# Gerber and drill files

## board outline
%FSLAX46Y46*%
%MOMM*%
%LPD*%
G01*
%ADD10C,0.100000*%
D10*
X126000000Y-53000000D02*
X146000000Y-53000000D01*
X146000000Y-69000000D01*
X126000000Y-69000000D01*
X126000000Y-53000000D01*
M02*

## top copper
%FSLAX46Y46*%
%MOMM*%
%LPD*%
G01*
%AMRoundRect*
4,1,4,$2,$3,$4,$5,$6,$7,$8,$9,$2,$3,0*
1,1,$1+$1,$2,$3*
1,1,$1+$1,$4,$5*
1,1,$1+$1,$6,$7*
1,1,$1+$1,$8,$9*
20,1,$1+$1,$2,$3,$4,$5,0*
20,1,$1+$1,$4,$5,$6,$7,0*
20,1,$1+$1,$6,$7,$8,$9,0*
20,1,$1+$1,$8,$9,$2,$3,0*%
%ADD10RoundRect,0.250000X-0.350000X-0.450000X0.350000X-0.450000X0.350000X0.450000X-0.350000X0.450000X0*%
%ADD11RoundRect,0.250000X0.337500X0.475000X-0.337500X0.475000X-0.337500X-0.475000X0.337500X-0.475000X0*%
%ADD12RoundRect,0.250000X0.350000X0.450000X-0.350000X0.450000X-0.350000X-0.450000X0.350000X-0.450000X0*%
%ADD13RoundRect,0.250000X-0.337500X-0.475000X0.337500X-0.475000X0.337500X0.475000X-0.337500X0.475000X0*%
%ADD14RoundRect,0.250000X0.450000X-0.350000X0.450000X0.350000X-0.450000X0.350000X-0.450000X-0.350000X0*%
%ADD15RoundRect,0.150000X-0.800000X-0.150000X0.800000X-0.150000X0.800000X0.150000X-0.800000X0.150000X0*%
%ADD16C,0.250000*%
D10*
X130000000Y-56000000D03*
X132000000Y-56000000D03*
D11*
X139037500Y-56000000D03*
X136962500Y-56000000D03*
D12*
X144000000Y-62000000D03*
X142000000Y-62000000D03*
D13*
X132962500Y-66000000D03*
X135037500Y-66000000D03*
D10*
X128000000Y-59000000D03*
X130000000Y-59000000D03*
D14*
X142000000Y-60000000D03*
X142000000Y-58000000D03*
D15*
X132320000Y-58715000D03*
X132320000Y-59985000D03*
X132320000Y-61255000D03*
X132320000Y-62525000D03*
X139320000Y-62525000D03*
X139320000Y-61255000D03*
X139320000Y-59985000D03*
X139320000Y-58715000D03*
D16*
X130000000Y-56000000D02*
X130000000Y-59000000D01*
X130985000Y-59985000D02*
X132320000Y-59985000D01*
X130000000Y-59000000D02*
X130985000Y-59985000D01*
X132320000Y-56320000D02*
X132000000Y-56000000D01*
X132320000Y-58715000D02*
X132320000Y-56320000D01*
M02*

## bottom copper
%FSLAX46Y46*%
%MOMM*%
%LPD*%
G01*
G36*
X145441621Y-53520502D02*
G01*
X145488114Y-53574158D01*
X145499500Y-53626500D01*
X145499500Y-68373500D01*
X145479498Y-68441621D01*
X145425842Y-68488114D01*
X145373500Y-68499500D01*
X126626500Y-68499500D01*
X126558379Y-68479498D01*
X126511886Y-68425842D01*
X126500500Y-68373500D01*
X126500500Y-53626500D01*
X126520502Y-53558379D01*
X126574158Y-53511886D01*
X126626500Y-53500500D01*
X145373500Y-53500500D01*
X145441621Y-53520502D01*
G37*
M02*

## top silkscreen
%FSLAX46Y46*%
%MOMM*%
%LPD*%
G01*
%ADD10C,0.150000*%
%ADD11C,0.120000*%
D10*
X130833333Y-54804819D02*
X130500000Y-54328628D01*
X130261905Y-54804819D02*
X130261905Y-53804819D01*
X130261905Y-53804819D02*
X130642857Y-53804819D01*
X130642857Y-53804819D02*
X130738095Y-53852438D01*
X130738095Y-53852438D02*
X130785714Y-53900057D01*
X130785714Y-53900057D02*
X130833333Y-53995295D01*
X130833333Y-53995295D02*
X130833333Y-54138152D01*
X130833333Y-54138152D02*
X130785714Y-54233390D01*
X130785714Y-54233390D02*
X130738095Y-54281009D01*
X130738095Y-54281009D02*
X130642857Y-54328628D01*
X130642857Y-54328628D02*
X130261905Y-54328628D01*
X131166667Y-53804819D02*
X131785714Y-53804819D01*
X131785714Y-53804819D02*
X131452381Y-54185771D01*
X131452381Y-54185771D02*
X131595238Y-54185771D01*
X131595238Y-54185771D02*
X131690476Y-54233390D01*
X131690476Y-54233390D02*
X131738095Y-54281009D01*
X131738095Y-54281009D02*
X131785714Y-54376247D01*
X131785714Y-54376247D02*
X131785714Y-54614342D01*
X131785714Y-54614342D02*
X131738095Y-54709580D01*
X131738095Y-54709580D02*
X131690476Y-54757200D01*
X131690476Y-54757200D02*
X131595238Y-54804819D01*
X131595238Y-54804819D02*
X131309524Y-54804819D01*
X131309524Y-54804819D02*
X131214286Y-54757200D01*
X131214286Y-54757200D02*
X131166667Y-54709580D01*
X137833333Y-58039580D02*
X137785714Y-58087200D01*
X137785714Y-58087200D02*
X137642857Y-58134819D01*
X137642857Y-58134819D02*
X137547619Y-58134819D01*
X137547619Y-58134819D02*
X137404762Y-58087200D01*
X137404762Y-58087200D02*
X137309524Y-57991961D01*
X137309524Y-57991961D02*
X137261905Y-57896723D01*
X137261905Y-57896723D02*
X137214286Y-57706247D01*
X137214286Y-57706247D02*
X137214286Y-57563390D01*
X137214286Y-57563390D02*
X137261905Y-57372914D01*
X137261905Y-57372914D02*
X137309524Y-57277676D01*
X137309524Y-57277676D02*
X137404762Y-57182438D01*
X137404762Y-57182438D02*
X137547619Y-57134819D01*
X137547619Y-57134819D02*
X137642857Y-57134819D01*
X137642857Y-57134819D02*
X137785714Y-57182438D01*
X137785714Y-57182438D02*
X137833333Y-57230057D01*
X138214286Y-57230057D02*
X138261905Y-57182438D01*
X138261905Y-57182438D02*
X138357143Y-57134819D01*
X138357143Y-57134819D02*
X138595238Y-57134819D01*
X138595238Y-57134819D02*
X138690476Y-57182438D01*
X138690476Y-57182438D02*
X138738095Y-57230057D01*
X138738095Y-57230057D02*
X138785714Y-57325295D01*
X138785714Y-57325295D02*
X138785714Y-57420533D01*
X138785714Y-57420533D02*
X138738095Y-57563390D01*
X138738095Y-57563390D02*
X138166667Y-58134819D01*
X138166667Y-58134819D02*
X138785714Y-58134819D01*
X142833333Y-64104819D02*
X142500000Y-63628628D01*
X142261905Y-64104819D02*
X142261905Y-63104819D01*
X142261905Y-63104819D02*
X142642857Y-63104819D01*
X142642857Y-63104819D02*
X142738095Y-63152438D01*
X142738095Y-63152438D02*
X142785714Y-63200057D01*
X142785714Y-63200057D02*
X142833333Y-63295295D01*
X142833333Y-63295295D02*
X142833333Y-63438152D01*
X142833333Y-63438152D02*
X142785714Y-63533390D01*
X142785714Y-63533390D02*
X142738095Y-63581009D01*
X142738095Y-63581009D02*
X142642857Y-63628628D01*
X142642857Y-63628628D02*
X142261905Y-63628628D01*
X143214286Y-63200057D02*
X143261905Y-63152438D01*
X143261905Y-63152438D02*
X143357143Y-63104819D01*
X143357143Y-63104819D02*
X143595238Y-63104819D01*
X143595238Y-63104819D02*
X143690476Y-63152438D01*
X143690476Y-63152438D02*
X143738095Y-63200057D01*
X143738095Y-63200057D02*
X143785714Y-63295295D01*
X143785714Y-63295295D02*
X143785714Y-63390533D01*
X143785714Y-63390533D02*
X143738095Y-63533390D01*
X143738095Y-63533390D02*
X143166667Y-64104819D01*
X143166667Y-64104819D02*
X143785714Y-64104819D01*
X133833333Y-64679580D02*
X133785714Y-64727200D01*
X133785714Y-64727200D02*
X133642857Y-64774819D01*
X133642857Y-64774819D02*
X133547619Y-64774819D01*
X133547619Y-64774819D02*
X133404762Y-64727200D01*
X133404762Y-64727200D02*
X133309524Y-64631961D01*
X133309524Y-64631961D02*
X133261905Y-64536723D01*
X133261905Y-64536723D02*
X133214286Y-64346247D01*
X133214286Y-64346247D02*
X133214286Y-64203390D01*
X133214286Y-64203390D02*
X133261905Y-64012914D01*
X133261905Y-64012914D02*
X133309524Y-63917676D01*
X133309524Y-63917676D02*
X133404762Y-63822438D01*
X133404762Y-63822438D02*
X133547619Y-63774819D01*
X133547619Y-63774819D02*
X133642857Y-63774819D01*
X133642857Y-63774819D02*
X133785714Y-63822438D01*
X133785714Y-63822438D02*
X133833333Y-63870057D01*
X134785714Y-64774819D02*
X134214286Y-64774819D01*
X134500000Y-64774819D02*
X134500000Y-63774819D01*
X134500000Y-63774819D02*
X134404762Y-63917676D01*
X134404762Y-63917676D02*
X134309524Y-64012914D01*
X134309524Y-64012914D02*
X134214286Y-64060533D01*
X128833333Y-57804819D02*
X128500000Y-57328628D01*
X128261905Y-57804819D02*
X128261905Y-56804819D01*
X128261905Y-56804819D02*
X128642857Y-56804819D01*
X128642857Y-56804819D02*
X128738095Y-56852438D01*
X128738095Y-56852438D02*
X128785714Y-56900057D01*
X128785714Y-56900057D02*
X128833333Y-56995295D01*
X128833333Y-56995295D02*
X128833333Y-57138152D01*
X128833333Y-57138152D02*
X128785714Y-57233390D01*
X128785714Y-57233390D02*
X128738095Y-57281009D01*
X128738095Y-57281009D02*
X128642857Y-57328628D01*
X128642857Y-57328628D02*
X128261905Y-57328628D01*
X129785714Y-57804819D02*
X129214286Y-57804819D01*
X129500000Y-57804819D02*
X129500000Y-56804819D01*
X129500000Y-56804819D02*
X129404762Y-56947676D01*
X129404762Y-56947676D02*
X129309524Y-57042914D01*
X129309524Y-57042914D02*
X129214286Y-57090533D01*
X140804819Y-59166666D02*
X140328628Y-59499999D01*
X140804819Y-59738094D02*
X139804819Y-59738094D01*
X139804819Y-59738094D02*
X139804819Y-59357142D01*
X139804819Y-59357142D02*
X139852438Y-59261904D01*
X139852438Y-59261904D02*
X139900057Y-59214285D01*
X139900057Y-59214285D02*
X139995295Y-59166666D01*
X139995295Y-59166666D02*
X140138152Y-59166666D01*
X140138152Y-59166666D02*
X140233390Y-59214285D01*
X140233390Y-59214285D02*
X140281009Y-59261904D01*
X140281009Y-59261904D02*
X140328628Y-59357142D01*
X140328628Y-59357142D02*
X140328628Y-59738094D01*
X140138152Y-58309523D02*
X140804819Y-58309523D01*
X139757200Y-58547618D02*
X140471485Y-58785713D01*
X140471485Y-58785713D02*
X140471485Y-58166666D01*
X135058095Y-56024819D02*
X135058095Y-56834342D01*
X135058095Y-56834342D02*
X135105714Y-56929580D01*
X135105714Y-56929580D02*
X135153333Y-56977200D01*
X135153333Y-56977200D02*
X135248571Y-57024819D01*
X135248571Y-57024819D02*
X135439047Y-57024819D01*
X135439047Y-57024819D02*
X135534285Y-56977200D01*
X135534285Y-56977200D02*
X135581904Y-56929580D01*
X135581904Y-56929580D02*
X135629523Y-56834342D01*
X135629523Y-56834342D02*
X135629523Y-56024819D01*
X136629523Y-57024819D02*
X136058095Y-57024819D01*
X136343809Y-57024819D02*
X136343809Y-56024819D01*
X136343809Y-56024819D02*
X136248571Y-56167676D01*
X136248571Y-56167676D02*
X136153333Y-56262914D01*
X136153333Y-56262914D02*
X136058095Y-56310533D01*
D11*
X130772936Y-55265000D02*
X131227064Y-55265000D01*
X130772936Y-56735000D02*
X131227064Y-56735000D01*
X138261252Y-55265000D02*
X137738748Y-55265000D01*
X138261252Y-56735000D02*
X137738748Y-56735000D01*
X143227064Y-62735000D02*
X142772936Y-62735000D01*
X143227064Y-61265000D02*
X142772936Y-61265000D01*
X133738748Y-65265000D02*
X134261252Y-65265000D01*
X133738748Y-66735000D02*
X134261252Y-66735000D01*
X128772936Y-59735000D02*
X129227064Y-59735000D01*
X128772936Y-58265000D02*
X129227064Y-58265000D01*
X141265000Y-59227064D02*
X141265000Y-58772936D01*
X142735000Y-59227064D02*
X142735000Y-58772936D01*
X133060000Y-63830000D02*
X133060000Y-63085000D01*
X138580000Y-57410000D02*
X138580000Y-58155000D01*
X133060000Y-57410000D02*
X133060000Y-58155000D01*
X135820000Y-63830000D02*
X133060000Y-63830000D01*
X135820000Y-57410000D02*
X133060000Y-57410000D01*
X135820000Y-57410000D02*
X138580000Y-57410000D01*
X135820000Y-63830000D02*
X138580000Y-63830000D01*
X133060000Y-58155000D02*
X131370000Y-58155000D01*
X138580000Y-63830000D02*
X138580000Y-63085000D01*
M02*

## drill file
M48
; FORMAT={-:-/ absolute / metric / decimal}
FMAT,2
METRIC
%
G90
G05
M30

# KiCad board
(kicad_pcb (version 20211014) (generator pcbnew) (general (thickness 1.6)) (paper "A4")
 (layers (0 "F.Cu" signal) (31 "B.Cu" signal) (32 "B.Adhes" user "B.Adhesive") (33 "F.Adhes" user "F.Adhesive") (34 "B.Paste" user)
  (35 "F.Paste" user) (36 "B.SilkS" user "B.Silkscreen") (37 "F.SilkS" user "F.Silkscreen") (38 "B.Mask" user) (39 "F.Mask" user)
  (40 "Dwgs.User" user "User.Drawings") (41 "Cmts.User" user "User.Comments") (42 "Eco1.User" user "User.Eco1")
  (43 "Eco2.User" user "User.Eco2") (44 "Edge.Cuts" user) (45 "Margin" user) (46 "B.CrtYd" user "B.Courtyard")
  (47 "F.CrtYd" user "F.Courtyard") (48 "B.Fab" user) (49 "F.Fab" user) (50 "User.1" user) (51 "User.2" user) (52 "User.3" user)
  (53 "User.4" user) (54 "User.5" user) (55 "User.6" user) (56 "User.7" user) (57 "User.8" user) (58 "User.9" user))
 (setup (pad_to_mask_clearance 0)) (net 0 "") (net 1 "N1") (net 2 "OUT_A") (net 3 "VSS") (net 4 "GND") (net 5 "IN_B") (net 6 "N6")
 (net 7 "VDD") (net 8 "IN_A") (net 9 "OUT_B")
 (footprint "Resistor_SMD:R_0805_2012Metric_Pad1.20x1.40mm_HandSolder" (layer "F.Cu") (at 131 56)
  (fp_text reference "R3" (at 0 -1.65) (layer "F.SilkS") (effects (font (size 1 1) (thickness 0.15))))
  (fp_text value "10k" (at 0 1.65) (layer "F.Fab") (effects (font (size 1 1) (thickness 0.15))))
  (fp_line (start -0.227064 -0.735) (end 0.227064 -0.735) (layer "F.SilkS") (width 0.12))
  (fp_line (start -0.227064 0.735) (end 0.227064 0.735) (layer "F.SilkS") (width 0.12))
  (pad "1" smd roundrect (at -1 0) (size 1.2 1.4) (layers "F.Cu" "F.Paste" "F.Mask") (roundrect_rratio 0.208333) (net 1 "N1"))
  (pad "2" smd roundrect (at 1 0) (size 1.2 1.4) (layers "F.Cu" "F.Paste" "F.Mask") (roundrect_rratio 0.208333) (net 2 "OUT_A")))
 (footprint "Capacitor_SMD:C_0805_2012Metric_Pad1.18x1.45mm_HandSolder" (layer "F.Cu") (at 138 56 180)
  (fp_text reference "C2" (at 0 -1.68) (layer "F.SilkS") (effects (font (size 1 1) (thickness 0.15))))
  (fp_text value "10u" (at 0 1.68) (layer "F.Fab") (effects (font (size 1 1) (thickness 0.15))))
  (fp_line (start -0.261252 0.735) (end 0.261252 0.735) (layer "F.SilkS") (width 0.12))
  (fp_line (start -0.261252 -0.735) (end 0.261252 -0.735) (layer "F.SilkS") (width 0.12))
  (pad "1" smd roundrect (at -1.0375 0 180) (size 1.175 1.45) (layers "F.Cu" "F.Paste" "F.Mask") (roundrect_rratio 0.212766) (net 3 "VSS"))
  (pad "2" smd roundrect (at 1.0375 0 180) (size 1.175 1.45) (layers "F.Cu" "F.Paste" "F.Mask") (roundrect_rratio 0.212766) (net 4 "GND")))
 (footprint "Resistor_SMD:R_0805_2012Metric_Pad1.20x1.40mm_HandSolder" (layer "F.Cu") (at 143 62 180)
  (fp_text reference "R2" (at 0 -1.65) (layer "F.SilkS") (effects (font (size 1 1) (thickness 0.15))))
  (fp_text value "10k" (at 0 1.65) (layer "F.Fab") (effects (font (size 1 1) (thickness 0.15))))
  (fp_line (start -0.227064 -0.735) (end 0.227064 -0.735) (layer "F.SilkS") (width 0.12))
  (fp_line (start -0.227064 0.735) (end 0.227064 0.735) (layer "F.SilkS") (width 0.12))
  (pad "1" smd roundrect (at -1 0 180) (size 1.2 1.4) (layers "F.Cu" "F.Paste" "F.Mask") (roundrect_rratio 0.208333) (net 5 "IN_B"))
  (pad "2" smd roundrect (at 1 0 180) (size 1.2 1.4) (layers "F.Cu" "F.Paste" "F.Mask") (roundrect_rratio 0.208333) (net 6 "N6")))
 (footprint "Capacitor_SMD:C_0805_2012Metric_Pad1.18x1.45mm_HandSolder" (layer "F.Cu") (at 134 66)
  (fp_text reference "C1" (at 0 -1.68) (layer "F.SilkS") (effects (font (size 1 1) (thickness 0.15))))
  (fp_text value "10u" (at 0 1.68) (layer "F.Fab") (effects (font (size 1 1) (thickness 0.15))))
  (fp_line (start -0.261252 -0.735) (end 0.261252 -0.735) (layer "F.SilkS") (width 0.12))
  (fp_line (start -0.261252 0.735) (end 0.261252 0.735) (layer "F.SilkS") (width 0.12))
  (pad "1" smd roundrect (at -1.0375 0) (size 1.175 1.45) (layers "F.Cu" "F.Paste" "F.Mask") (roundrect_rratio 0.212766) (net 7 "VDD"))
  (pad "2" smd roundrect (at 1.0375 0) (size 1.175 1.45) (layers "F.Cu" "F.Paste" "F.Mask") (roundrect_rratio 0.212766) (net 4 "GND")))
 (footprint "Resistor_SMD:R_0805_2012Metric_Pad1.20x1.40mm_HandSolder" (layer "F.Cu") (at 129 59)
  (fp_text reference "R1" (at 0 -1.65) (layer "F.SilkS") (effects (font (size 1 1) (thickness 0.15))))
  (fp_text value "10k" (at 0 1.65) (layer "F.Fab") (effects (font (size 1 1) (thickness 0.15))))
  (fp_line (start -0.227064 0.735) (end 0.227064 0.735) (layer "F.SilkS") (width 0.12))
  (fp_line (start -0.227064 -0.735) (end 0.227064 -0.735) (layer "F.SilkS") (width 0.12))
  (pad "1" smd roundrect (at -1 0) (size 1.2 1.4) (layers "F.Cu" "F.Paste" "F.Mask") (roundrect_rratio 0.208333) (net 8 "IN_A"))
  (pad "2" smd roundrect (at 1 0) (size 1.2 1.4) (layers "F.Cu" "F.Paste" "F.Mask") (roundrect_rratio 0.208333) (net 1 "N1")))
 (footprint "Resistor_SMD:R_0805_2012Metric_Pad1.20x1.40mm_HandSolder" (layer "F.Cu") (at 142 59 90)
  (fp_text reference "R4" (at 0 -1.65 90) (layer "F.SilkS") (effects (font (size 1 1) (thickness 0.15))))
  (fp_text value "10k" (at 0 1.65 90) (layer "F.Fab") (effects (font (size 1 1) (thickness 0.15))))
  (fp_line (start -0.227064 -0.735) (end 0.227064 -0.735) (layer "F.SilkS") (width 0.12))
  (fp_line (start -0.227064 0.735) (end 0.227064 0.735) (layer "F.SilkS") (width 0.12))
  (pad "1" smd roundrect (at -1 0 90) (size 1.2 1.4) (layers "F.Cu" "F.Paste" "F.Mask") (roundrect_rratio 0.208333) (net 6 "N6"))
  (pad "2" smd roundrect (at 1 0 90) (size 1.2 1.4) (layers "F.Cu" "F.Paste" "F.Mask") (roundrect_rratio 0.208333) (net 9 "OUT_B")))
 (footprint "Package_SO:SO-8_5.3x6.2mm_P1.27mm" (layer "F.Cu") (at 135.82 60.62)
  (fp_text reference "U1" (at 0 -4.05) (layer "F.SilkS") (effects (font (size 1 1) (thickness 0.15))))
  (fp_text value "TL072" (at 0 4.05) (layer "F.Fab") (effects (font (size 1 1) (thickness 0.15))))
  (fp_line (start -2.76 3.21) (end -2.76 2.465) (layer "F.SilkS") (width 0.12))
  (fp_line (start 2.76 -3.21) (end 2.76 -2.465) (layer "F.SilkS") (width 0.12))
  (fp_line (start -2.76 -3.21) (end -2.76 -2.465) (layer "F.SilkS") (width 0.12))
  (fp_line (start 0 3.21) (end -2.76 3.21) (layer "F.SilkS") (width 0.12))
  (fp_line (start 0 -3.21) (end -2.76 -3.21) (layer "F.SilkS") (width 0.12))
  (fp_line (start 0 -3.21) (end 2.76 -3.21) (layer "F.SilkS") (width 0.12))
  (fp_line (start 0 3.21) (end 2.76 3.21) (layer "F.SilkS") (width 0.12))
  (fp_line (start -2.76 -2.465) (end -4.45 -2.465) (layer "F.SilkS") (width 0.12))
  (fp_line (start 2.76 3.21) (end 2.76 2.465) (layer "F.SilkS") (width 0.12))
  (pad "1" smd roundrect (at -3.5 -1.905) (size 1.9 0.6) (layers "F.Cu" "F.Paste" "F.Mask") (roundrect_rratio 0.25) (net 2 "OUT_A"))
  (pad "2" smd roundrect (at -3.5 -0.635) (size 1.9 0.6) (layers "F.Cu" "F.Paste" "F.Mask") (roundrect_rratio 0.25) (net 1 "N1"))
  (pad "3" smd roundrect (at -3.5 0.635) (size 1.9 0.6) (layers "F.Cu" "F.Paste" "F.Mask") (roundrect_rratio 0.25) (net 4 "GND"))
  (pad "4" smd roundrect (at -3.5 1.905) (size 1.9 0.6) (layers "F.Cu" "F.Paste" "F.Mask") (roundrect_rratio 0.25) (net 7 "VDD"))
  (pad "5" smd roundrect (at 3.5 1.905) (size 1.9 0.6) (layers "F.Cu" "F.Paste" "F.Mask") (roundrect_rratio 0.25) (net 4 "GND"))
  (pad "6" smd roundrect (at 3.5 0.635) (size 1.9 0.6) (layers "F.Cu" "F.Paste" "F.Mask") (roundrect_rratio 0.25) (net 6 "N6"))
  (pad "7" smd roundrect (at 3.5 -0.635) (size 1.9 0.6) (layers "F.Cu" "F.Paste" "F.Mask") (roundrect_rratio 0.25) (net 9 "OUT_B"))
  (pad "8" smd roundrect (at 3.5 -1.905) (size 1.9 0.6) (layers "F.Cu" "F.Paste" "F.Mask") (roundrect_rratio 0.25) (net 3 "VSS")))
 (gr_rect (start 126 53) (end 146 69) (layer "Edge.Cuts") (width 0.1) (fill none))
 (segment (start 130 56) (end 130 59) (width 0.25) (layer "F.Cu") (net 1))
 (segment (start 130.985 59.985) (end 132.32 59.985) (width 0.25) (layer "F.Cu") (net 1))
 (segment (start 130 59) (end 130.985 59.985) (width 0.25) (layer "F.Cu") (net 1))
 (segment (start 132.32 56.32) (end 132 56) (width 0.25) (layer "F.Cu") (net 2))
 (segment (start 132.32 58.715) (end 132.32 56.32) (width 0.25) (layer "F.Cu") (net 2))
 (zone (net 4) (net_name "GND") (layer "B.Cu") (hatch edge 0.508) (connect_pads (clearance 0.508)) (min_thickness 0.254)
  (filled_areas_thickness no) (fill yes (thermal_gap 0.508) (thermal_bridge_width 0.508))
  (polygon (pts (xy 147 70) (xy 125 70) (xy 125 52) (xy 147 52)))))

